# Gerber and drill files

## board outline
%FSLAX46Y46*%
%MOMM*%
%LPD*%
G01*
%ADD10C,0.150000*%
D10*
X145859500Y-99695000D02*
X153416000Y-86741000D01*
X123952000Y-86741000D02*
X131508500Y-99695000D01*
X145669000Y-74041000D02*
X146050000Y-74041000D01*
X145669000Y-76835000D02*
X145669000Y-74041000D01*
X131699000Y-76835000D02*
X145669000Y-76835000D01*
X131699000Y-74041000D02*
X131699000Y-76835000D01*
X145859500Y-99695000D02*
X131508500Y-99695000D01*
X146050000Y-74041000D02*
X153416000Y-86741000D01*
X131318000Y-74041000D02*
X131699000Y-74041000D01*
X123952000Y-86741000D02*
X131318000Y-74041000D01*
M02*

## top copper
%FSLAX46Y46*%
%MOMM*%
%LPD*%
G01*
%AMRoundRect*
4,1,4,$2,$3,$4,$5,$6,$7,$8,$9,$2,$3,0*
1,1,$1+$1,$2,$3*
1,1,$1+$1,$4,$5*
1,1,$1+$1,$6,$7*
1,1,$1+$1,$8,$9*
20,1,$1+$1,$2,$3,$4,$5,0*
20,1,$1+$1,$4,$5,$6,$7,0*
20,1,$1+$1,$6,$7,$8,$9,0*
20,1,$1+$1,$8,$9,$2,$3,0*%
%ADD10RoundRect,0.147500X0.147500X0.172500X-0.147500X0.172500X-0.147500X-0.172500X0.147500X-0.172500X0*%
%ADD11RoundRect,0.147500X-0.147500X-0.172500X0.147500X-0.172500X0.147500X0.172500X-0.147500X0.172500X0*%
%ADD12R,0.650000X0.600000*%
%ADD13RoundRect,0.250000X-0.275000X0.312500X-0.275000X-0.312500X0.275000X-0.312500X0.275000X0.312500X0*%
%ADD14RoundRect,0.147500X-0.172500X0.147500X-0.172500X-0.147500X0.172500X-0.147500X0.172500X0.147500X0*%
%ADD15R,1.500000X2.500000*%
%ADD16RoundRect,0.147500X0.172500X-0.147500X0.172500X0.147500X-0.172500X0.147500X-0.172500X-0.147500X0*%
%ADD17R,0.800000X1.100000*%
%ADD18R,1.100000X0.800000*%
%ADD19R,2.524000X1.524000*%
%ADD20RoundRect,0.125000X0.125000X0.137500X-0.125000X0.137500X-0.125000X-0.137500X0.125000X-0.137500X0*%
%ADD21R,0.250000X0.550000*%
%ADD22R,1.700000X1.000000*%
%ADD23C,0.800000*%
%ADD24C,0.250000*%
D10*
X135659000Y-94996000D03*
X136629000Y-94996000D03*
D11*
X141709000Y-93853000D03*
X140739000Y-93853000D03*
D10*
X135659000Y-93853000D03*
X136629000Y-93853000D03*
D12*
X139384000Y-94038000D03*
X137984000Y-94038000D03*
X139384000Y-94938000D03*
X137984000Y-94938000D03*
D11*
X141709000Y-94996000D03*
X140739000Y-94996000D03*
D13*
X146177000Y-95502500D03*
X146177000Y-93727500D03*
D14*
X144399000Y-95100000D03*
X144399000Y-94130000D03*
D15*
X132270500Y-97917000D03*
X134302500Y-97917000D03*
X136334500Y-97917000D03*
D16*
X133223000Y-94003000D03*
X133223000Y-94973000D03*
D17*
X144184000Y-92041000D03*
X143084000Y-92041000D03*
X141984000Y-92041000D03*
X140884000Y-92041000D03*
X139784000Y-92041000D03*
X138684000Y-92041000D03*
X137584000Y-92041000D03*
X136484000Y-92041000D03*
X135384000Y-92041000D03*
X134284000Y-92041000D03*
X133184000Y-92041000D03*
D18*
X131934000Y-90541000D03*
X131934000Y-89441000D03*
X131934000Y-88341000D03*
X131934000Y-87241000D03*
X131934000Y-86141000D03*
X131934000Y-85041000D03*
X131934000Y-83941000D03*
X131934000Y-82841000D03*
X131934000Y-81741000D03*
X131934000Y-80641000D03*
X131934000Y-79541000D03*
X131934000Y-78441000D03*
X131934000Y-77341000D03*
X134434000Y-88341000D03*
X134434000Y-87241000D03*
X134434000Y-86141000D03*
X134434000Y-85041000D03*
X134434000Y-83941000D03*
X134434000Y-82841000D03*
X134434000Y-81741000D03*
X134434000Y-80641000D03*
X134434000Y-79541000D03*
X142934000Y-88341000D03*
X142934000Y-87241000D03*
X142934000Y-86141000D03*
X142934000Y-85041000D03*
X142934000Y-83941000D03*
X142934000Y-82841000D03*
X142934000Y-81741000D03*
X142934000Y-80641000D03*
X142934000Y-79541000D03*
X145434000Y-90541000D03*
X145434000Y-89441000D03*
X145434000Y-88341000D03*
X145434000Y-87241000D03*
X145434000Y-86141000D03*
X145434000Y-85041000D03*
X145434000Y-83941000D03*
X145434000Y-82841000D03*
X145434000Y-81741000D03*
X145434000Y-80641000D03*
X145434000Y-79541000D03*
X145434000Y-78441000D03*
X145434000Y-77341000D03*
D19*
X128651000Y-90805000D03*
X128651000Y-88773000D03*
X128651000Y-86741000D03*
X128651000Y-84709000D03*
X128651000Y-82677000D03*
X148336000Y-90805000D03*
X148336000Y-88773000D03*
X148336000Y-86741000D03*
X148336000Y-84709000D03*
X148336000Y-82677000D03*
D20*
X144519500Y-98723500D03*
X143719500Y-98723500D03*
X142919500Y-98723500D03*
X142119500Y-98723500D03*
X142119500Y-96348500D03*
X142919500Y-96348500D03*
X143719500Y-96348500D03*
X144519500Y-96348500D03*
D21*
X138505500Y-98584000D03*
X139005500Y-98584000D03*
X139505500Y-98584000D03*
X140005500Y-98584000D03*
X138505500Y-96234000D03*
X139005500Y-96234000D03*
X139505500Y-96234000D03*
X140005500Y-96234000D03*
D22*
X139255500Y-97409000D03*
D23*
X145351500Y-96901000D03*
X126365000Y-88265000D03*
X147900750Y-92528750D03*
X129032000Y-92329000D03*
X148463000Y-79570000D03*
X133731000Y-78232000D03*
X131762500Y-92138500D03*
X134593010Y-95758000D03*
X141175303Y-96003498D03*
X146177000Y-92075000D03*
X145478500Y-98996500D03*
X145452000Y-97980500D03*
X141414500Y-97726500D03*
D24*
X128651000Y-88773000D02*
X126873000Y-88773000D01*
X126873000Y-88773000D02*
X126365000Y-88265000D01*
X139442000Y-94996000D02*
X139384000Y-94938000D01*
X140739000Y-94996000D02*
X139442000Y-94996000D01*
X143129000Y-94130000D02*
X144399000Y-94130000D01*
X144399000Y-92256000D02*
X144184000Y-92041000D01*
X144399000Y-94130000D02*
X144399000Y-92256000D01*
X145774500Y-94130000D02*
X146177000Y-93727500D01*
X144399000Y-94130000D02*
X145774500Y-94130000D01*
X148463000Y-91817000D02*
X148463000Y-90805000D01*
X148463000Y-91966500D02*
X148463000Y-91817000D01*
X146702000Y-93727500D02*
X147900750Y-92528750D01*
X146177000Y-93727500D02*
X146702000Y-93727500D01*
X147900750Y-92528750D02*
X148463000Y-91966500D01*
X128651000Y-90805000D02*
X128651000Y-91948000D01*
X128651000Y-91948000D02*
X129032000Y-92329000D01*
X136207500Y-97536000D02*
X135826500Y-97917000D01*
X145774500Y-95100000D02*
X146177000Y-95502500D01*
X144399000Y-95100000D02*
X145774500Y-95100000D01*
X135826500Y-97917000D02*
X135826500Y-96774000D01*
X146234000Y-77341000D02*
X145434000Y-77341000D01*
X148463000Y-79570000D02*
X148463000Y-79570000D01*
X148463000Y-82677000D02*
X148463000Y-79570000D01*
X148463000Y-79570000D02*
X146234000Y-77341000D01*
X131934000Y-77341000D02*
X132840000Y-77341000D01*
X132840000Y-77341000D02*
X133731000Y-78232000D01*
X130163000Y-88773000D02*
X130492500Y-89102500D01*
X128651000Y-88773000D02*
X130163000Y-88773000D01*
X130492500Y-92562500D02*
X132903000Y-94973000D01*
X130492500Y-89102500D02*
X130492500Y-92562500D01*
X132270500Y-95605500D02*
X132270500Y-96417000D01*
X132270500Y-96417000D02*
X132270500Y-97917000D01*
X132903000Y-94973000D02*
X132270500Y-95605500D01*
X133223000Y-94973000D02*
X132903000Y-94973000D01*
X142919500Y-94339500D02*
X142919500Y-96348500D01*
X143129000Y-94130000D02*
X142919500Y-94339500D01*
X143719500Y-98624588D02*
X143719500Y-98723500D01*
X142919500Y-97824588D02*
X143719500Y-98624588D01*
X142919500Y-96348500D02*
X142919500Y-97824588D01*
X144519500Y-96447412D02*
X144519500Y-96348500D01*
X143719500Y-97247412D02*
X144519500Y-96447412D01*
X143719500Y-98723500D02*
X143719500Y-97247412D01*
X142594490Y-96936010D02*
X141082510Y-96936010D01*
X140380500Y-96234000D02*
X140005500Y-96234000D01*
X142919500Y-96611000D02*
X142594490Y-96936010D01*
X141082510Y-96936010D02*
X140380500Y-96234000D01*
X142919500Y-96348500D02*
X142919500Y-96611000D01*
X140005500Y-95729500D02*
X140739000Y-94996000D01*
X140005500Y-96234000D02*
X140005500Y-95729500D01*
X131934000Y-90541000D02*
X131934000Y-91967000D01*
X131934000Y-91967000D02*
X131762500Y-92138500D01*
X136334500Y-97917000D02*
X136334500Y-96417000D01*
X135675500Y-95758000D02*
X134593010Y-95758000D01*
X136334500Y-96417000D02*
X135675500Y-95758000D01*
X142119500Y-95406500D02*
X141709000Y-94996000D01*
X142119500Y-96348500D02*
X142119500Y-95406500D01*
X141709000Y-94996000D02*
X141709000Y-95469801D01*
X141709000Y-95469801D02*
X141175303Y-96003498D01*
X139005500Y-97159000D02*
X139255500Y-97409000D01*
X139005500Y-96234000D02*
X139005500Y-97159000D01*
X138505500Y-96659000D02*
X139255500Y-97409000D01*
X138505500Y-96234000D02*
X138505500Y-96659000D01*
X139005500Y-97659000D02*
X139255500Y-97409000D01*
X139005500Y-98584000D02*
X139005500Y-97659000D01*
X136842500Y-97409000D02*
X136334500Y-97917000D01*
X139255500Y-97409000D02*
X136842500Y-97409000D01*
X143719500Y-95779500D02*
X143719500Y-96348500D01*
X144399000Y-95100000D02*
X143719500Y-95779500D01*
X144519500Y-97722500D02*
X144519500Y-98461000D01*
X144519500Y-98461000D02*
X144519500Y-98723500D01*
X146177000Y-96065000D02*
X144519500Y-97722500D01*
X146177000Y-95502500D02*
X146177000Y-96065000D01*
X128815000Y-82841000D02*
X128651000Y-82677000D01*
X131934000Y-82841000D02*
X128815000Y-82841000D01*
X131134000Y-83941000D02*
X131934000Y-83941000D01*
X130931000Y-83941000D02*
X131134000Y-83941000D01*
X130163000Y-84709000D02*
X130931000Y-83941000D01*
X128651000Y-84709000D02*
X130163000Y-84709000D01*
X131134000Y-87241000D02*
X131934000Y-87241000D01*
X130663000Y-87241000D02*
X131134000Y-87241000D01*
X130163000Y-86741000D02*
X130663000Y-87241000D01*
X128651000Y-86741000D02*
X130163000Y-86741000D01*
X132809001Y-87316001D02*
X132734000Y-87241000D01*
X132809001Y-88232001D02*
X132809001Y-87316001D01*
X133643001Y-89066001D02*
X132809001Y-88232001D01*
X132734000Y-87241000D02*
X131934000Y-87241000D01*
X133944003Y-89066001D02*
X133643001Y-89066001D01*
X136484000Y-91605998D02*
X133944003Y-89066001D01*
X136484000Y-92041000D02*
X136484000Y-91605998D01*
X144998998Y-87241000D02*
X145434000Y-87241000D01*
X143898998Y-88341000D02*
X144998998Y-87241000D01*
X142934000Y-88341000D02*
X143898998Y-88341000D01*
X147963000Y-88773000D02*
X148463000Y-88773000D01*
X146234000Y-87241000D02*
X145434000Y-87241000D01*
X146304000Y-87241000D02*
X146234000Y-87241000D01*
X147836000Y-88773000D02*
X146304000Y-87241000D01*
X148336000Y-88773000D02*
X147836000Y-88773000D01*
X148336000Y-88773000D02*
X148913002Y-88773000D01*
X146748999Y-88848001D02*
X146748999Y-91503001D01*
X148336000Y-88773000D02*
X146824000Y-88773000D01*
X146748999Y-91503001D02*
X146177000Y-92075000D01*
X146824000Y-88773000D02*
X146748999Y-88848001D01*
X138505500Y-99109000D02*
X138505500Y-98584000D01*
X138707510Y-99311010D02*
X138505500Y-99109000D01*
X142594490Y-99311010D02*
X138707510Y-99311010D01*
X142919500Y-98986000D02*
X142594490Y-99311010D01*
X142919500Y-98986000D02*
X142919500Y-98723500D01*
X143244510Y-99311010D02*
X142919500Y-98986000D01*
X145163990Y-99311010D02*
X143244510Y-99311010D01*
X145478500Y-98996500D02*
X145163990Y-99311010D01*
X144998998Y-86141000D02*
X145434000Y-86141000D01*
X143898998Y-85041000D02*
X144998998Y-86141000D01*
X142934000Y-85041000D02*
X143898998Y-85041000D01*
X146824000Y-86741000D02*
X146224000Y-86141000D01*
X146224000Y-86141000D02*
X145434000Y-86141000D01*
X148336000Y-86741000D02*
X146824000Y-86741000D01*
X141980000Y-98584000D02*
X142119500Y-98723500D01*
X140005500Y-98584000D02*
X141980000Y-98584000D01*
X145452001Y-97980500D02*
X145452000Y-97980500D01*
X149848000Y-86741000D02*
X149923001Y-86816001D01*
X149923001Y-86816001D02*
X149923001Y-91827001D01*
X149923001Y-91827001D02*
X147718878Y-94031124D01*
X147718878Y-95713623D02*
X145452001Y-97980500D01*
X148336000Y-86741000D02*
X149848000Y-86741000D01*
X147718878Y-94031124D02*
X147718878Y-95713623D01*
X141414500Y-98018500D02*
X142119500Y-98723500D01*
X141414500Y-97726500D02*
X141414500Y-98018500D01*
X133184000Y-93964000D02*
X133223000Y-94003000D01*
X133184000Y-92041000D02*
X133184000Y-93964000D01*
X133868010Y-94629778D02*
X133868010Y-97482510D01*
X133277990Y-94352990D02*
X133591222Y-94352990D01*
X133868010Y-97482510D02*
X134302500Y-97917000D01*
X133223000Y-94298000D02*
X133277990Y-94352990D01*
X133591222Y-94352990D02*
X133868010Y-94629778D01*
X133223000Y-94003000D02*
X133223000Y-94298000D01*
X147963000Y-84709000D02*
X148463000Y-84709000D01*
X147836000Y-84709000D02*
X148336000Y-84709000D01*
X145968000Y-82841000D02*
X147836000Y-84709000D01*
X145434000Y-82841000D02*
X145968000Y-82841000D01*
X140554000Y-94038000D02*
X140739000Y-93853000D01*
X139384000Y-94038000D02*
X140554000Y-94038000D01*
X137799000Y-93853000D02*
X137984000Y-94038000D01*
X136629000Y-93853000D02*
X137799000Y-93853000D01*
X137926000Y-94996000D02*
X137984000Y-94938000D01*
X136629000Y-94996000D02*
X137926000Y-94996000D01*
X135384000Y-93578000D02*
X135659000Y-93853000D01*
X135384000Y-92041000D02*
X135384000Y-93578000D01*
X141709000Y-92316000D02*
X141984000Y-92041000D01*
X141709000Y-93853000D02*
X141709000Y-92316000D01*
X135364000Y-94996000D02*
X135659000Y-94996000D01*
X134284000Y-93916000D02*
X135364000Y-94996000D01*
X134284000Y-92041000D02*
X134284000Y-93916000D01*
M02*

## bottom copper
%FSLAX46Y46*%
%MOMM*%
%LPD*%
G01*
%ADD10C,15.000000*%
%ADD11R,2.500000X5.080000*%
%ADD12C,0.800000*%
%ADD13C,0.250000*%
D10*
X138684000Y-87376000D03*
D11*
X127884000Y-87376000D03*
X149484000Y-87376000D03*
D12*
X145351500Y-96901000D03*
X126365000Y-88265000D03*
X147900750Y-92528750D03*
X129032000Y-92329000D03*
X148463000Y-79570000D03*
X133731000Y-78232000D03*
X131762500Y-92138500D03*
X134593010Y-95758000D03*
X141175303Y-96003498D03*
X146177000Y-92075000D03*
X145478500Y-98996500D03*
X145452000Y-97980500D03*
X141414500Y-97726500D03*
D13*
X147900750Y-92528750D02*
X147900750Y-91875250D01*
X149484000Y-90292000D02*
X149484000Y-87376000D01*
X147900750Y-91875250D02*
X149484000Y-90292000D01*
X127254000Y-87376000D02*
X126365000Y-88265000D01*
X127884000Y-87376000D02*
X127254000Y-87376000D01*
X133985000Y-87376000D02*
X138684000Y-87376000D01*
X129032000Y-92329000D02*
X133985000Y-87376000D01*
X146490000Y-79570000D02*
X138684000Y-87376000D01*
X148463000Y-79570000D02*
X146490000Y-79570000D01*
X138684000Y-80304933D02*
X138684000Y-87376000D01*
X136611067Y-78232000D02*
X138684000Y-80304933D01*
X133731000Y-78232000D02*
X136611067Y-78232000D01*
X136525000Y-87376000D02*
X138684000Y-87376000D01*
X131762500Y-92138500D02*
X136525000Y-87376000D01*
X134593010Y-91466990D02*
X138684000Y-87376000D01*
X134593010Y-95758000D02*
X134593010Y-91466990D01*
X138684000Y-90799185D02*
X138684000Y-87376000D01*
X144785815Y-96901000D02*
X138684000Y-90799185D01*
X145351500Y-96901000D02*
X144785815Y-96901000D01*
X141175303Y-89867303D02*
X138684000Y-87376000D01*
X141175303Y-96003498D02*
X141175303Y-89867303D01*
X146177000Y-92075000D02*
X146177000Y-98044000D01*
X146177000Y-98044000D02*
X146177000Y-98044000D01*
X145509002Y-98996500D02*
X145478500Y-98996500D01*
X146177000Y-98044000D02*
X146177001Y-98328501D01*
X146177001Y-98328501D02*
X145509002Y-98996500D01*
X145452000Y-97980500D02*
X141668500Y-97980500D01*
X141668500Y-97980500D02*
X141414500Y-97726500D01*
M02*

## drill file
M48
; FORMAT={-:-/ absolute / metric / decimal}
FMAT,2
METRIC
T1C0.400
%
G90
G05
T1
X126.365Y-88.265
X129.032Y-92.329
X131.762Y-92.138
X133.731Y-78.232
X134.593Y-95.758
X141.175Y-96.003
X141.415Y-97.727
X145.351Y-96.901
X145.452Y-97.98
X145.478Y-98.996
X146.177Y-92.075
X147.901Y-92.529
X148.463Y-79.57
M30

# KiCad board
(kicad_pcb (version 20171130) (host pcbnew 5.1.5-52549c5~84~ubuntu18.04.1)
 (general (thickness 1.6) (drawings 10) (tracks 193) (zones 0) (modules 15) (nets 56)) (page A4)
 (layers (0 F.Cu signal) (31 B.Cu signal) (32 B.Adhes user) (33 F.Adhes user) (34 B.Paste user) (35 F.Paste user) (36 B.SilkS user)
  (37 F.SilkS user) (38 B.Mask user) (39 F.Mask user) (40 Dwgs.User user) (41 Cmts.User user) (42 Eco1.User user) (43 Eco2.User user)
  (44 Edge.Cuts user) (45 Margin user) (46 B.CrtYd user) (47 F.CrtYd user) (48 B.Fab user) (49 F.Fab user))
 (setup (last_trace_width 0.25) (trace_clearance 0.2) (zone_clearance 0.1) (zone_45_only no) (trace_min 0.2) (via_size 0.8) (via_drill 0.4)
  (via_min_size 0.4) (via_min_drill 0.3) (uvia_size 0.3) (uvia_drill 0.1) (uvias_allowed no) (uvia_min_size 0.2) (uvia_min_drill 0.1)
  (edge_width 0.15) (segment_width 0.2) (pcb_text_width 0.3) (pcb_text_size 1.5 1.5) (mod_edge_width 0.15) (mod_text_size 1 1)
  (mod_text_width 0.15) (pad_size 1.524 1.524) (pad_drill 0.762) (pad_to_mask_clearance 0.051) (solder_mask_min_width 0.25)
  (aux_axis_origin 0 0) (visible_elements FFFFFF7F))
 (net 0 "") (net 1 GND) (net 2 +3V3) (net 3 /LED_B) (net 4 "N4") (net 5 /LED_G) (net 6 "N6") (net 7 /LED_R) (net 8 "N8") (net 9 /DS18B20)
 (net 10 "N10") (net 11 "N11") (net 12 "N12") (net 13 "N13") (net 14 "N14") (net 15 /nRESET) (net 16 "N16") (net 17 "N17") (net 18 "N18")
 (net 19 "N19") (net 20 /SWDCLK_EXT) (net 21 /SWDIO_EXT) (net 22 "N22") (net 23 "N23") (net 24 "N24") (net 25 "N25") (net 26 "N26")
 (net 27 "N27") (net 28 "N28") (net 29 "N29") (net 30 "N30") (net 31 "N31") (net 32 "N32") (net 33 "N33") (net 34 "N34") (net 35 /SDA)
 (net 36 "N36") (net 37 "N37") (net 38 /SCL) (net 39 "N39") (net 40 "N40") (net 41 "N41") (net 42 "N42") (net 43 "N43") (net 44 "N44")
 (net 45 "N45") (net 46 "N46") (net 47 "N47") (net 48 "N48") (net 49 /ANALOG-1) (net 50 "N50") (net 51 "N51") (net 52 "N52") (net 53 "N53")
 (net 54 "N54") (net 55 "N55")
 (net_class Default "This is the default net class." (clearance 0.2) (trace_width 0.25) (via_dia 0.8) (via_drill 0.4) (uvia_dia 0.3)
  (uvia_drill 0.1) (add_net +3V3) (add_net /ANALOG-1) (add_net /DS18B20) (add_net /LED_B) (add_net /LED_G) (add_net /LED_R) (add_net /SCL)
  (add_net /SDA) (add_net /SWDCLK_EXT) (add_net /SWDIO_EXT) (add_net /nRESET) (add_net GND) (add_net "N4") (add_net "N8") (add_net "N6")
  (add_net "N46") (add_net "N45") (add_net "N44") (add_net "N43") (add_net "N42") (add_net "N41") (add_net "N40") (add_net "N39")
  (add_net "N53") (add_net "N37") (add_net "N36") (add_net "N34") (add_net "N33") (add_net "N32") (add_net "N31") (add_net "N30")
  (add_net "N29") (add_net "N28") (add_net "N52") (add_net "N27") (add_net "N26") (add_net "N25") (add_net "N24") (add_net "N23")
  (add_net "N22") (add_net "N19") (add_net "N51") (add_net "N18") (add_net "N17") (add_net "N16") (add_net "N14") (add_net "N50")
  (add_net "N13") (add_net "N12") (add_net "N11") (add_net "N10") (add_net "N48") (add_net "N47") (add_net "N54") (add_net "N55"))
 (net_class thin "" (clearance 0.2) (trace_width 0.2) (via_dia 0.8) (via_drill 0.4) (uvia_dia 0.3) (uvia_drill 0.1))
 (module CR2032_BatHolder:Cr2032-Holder (layer B.Cu) (at 138.684 87.376)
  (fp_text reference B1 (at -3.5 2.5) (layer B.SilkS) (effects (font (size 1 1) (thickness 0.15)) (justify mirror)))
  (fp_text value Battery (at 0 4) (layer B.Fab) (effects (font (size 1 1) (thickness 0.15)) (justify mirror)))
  (pad 2 smd circle (at 0 0) (size 15 15) (layers B.Cu B.Mask) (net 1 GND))
  (pad 1 smd rect (at -10.8 0) (size 2.5 5.08) (layers B.Cu B.Paste B.Mask) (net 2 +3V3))
  (pad 1 smd rect (at 10.8 0) (size 2.5 5.08) (layers B.Cu B.Paste B.Mask) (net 2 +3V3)))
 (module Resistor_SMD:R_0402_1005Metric (layer F.Cu) (at 136.144 94.996 180)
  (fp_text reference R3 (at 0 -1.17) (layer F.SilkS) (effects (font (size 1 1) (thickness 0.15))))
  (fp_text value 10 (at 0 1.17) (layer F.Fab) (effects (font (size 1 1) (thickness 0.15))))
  (pad 2 smd roundrect (at 0.485 0 180) (size 0.59 0.64) (layers F.Cu F.Paste F.Mask) (roundrect_rratio 0.25) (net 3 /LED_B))
  (pad 1 smd roundrect (at -0.485 0 180) (size 0.59 0.64) (layers F.Cu F.Paste F.Mask) (roundrect_rratio 0.25) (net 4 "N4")))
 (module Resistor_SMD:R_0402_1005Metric (layer F.Cu) (at 141.224 93.853)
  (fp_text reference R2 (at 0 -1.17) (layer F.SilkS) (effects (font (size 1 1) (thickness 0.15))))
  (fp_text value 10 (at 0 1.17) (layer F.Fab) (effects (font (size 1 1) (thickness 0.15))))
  (pad 2 smd roundrect (at 0.485 0) (size 0.59 0.64) (layers F.Cu F.Paste F.Mask) (roundrect_rratio 0.25) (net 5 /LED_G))
  (pad 1 smd roundrect (at -0.485 0) (size 0.59 0.64) (layers F.Cu F.Paste F.Mask) (roundrect_rratio 0.25) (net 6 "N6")))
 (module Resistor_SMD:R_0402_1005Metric (layer F.Cu) (at 136.144 93.853 180)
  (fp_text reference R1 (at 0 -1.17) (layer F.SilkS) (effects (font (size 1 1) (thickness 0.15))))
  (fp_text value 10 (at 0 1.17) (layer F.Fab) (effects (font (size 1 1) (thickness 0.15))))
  (pad 2 smd roundrect (at 0.485 0 180) (size 0.59 0.64) (layers F.Cu F.Paste F.Mask) (roundrect_rratio 0.25) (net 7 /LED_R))
  (pad 1 smd roundrect (at -0.485 0 180) (size 0.59 0.64) (layers F.Cu F.Paste F.Mask) (roundrect_rratio 0.25) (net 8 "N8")))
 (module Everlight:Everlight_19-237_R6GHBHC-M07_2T (layer F.Cu) (at 138.684 94.488)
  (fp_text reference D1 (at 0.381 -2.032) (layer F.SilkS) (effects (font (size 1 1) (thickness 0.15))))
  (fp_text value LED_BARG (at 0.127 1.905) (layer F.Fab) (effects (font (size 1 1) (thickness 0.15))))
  (pad 4 smd rect (at 0.7 -0.45) (size 0.65 0.6) (layers F.Cu F.Paste F.Mask) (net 6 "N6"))
  (pad 3 smd rect (at -0.7 -0.45) (size 0.65 0.6) (layers F.Cu F.Paste F.Mask) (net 8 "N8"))
  (pad 2 smd rect (at 0.7 0.45) (size 0.65 0.6) (layers F.Cu F.Paste F.Mask) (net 2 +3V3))
  (pad 1 smd rect (at -0.7 0.45) (size 0.65 0.6) (layers F.Cu F.Paste F.Mask) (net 4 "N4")))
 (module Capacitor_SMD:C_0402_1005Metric (layer F.Cu) (at 141.224 94.996)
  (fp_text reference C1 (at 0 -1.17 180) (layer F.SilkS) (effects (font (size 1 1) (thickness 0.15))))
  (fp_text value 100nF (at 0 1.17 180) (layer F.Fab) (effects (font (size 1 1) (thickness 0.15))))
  (pad 2 smd roundrect (at 0.485 0) (size 0.59 0.64) (layers F.Cu F.Paste F.Mask) (roundrect_rratio 0.25) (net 1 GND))
  (pad 1 smd roundrect (at -0.485 0) (size 0.59 0.64) (layers F.Cu F.Paste F.Mask) (roundrect_rratio 0.25) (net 2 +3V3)))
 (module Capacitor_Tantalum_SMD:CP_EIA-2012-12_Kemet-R (layer F.Cu) (at 146.177 94.615 270)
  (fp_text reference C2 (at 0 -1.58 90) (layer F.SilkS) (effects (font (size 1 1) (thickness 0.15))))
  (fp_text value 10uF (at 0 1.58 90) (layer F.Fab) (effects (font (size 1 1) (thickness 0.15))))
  (pad 2 smd roundrect (at 0.8875 0 270) (size 1.125 1.05) (layers F.Cu F.Paste F.Mask) (roundrect_rratio 0.238095) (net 1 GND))
  (pad 1 smd roundrect (at -0.8875 0 270) (size 1.125 1.05) (layers F.Cu F.Paste F.Mask) (roundrect_rratio 0.238095) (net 2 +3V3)))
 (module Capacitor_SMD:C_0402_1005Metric (layer F.Cu) (at 144.399 94.615 270)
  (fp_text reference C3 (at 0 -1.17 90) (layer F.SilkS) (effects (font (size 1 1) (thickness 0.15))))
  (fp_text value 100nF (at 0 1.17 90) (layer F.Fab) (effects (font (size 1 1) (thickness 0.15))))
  (pad 2 smd roundrect (at 0.485 0 270) (size 0.59 0.64) (layers F.Cu F.Paste F.Mask) (roundrect_rratio 0.25) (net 1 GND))
  (pad 1 smd roundrect (at -0.485 0 270) (size 0.59 0.64) (layers F.Cu F.Paste F.Mask) (roundrect_rratio 0.25) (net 2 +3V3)))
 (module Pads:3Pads (layer F.Cu) (at 134.3025 100.457 180)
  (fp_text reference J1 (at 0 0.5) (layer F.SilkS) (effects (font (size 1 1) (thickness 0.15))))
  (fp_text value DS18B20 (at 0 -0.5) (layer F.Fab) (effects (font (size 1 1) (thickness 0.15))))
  (pad 3 smd rect (at 2.032 2.54 180) (size 1.5 2.5) (layers F.Cu F.Paste F.Mask) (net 2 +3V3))
  (pad 2 smd rect (at 0 2.54 180) (size 1.5 2.5) (layers F.Cu F.Paste F.Mask) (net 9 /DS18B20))
  (pad 1 smd rect (at -2.032 2.54 180) (size 1.5 2.5) (layers F.Cu F.Paste F.Mask) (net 1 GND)))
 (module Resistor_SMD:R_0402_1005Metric (layer F.Cu) (at 133.223 94.488 90)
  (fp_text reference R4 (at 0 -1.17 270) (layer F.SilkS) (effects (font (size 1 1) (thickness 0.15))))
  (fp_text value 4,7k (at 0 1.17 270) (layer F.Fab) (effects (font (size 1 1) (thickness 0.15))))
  (pad 2 smd roundrect (at 0.485 0 90) (size 0.59 0.64) (layers F.Cu F.Paste F.Mask) (roundrect_rratio 0.25) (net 9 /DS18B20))
  (pad 1 smd roundrect (at -0.485 0 90) (size 0.59 0.64) (layers F.Cu F.Paste F.Mask) (roundrect_rratio 0.25) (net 2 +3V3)))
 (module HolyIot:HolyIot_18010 (layer F.Cu) (at 138.684 74.041)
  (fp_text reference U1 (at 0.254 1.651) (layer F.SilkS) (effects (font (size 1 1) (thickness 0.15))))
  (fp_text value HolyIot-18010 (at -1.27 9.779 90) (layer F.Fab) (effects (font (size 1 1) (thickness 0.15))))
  (pad 55 smd rect (at 5.5 18) (size 0.8 1.1) (layers F.Cu F.Paste F.Mask) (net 2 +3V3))
  (pad 54 smd rect (at 4.4 18) (size 0.8 1.1) (layers F.Cu F.Paste F.Mask) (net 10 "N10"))
  (pad 53 smd rect (at 3.3 18) (size 0.8 1.1) (layers F.Cu F.Paste F.Mask) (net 5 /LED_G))
  (pad 52 smd rect (at 2.2 18) (size 0.8 1.1) (layers F.Cu F.Paste F.Mask) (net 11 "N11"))
  (pad 51 smd rect (at 1.1 18) (size 0.8 1.1) (layers F.Cu F.Paste F.Mask) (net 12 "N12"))
  (pad 50 smd rect (at 0 18) (size 0.8 1.1) (layers F.Cu F.Paste F.Mask) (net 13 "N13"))
  (pad 49 smd rect (at -1.1 18) (size 0.8 1.1) (layers F.Cu F.Paste F.Mask) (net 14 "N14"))
  (pad 48 smd rect (at -2.2 18) (size 0.8 1.1) (layers F.Cu F.Paste F.Mask) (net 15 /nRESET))
  (pad 47 smd rect (at -3.3 18) (size 0.8 1.1) (layers F.Cu F.Paste F.Mask) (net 7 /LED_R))
  (pad 46 smd rect (at -4.4 18) (size 0.8 1.1) (layers F.Cu F.Paste F.Mask) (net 3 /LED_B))
  (pad 45 smd rect (at -5.5 18) (size 0.8 1.1) (layers F.Cu F.Paste F.Mask) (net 9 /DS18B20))
  (pad 44 smd rect (at -6.75 16.5) (size 1.1 0.8) (layers F.Cu F.Paste F.Mask) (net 1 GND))
  (pad 43 smd rect (at -6.75 15.4) (size 1.1 0.8) (layers F.Cu F.Paste F.Mask) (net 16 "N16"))
  (pad 42 smd rect (at -6.75 14.3) (size 1.1 0.8) (layers F.Cu F.Paste F.Mask) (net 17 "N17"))
  (pad 41 smd rect (at -6.75 13.2) (size 1.1 0.8) (layers F.Cu F.Paste F.Mask) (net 15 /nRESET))
  (pad 40 smd rect (at -6.75 12.1) (size 1.1 0.8) (layers F.Cu F.Paste F.Mask) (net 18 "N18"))
  (pad 39 smd rect (at -6.75 11) (size 1.1 0.8) (layers F.Cu F.Paste F.Mask) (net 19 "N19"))
  (pad 38 smd rect (at -6.75 9.9) (size 1.1 0.8) (layers F.Cu F.Paste F.Mask) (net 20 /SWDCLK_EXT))
  (pad 37 smd rect (at -6.75 8.8) (size 1.1 0.8) (layers F.Cu F.Paste F.Mask) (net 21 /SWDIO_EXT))
  (pad 36 smd rect (at -6.75 7.7) (size 1.1 0.8) (layers F.Cu F.Paste F.Mask) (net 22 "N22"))
  (pad 35 smd rect (at -6.75 6.6) (size 1.1 0.8) (layers F.Cu F.Paste F.Mask) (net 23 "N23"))
  (pad 34 smd rect (at -6.75 5.5) (size 1.1 0.8) (layers F.Cu F.Paste F.Mask) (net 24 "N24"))
  (pad 33 smd rect (at -6.75 4.4) (size 1.1 0.8) (layers F.Cu F.Paste F.Mask) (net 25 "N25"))
  (pad 32 smd rect (at -6.75 3.3) (size 1.1 0.8) (layers F.Cu F.Paste F.Mask) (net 1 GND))
  (pad 31 smd rect (at -4.25 14.3) (size 1.1 0.8) (layers F.Cu F.Paste F.Mask) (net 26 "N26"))
  (pad 30 smd rect (at -4.25 13.2) (size 1.1 0.8) (layers F.Cu F.Paste F.Mask) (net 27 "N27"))
  (pad 29 smd rect (at -4.25 12.1) (size 1.1 0.8) (layers F.Cu F.Paste F.Mask) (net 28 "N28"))
  (pad 28 smd rect (at -4.25 11) (size 1.1 0.8) (layers F.Cu F.Paste F.Mask) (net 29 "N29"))
  (pad 27 smd rect (at -4.25 9.9) (size 1.1 0.8) (layers F.Cu F.Paste F.Mask) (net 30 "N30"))
  (pad 26 smd rect (at -4.25 8.8) (size 1.1 0.8) (layers F.Cu F.Paste F.Mask) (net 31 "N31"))
  (pad 25 smd rect (at -4.25 7.7) (size 1.1 0.8) (layers F.Cu F.Paste F.Mask) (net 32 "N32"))
  (pad 24 smd rect (at -4.25 6.6) (size 1.1 0.8) (layers F.Cu F.Paste F.Mask) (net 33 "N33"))
  (pad 23 smd rect (at -4.25 5.5) (size 1.1 0.8) (layers F.Cu F.Paste F.Mask) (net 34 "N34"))
  (pad 22 smd rect (at 4.25 14.3) (size 1.1 0.8) (layers F.Cu F.Paste F.Mask) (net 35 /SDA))
  (pad 21 smd rect (at 4.25 13.2) (size 1.1 0.8) (layers F.Cu F.Paste F.Mask) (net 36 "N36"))
  (pad 20 smd rect (at 4.25 12.1) (size 1.1 0.8) (layers F.Cu F.Paste F.Mask) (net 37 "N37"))
  (pad 19 smd rect (at 4.25 11) (size 1.1 0.8) (layers F.Cu F.Paste F.Mask) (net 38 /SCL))
  (pad 18 smd rect (at 4.25 9.9) (size 1.1 0.8) (layers F.Cu F.Paste F.Mask) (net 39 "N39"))
  (pad 17 smd rect (at 4.25 8.8) (size 1.1 0.8) (layers F.Cu F.Paste F.Mask) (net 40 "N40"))
  (pad 16 smd rect (at 4.25 7.7) (size 1.1 0.8) (layers F.Cu F.Paste F.Mask) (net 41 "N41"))
  (pad 15 smd rect (at 4.25 6.6) (size 1.1 0.8) (layers F.Cu F.Paste F.Mask) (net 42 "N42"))
  (pad 14 smd rect (at 4.25 5.5) (size 1.1 0.8) (layers F.Cu F.Paste F.Mask) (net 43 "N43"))
  (pad 13 smd rect (at 6.75 16.5) (size 1.1 0.8) (layers F.Cu F.Paste F.Mask) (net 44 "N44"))
  (pad 12 smd rect (at 6.75 15.4) (size 1.1 0.8) (layers F.Cu F.Paste F.Mask) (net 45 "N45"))
  (pad 11 smd rect (at 6.75 14.3) (size 1.1 0.8) (layers F.Cu F.Paste F.Mask) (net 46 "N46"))
  (pad 10 smd rect (at 6.75 13.2) (size 1.1 0.8) (layers F.Cu F.Paste F.Mask) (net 35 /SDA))
  (pad 9 smd rect (at 6.75 12.1) (size 1.1 0.8) (layers F.Cu F.Paste F.Mask) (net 38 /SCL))
  (pad 8 smd rect (at 6.75 11) (size 1.1 0.8) (layers F.Cu F.Paste F.Mask) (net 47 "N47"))
  (pad 7 smd rect (at 6.75 9.9) (size 1.1 0.8) (layers F.Cu F.Paste F.Mask) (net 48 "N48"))
  (pad 6 smd rect (at 6.75 8.8) (size 1.1 0.8) (layers F.Cu F.Paste F.Mask) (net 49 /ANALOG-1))
  (pad 5 smd rect (at 6.75 7.7) (size 1.1 0.8) (layers F.Cu F.Paste F.Mask) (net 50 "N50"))
  (pad 4 smd rect (at 6.75 6.6) (size 1.1 0.8) (layers F.Cu F.Paste F.Mask) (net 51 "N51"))
  (pad 3 smd rect (at 6.75 5.5) (size 1.1 0.8) (layers F.Cu F.Paste F.Mask) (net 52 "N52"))
  (pad 2 smd rect (at 6.75 4.4) (size 1.1 0.8) (layers F.Cu F.Paste F.Mask) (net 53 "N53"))
  (pad 1 smd rect (at 6.75 3.3) (size 1.1 0.8) (layers F.Cu F.Paste F.Mask) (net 1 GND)))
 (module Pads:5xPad (layer F.Cu) (at 128.651 82.677)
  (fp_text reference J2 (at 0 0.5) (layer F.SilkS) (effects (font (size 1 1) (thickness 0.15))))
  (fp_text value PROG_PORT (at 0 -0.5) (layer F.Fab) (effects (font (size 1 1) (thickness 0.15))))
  (pad 5 smd rect (at 0 8.128) (size 2.524 1.524) (layers F.Cu F.Paste F.Mask) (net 1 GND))
  (pad 4 smd rect (at 0 6.096) (size 2.524 1.524) (layers F.Cu F.Paste F.Mask) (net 2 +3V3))
  (pad 3 smd rect (at 0 4.064) (size 2.524 1.524) (layers F.Cu F.Paste F.Mask) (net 15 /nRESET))
  (pad 2 smd rect (at 0 2.032) (size 2.524 1.524) (layers F.Cu F.Paste F.Mask) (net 20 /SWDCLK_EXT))
  (pad 1 smd rect (at 0 0) (size 2.524 1.524) (layers F.Cu F.Paste F.Mask) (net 21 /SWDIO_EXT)))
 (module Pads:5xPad (layer F.Cu) (at 148.336 82.677)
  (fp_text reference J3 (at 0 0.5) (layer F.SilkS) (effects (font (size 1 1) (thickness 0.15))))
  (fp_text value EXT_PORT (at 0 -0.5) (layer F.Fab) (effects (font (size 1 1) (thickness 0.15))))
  (pad 5 smd rect (at 0 8.128) (size 2.524 1.524) (layers F.Cu F.Paste F.Mask) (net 2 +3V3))
  (pad 4 smd rect (at 0 6.096) (size 2.524 1.524) (layers F.Cu F.Paste F.Mask) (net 35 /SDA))
  (pad 3 smd rect (at 0 4.064) (size 2.524 1.524) (layers F.Cu F.Paste F.Mask) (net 38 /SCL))
  (pad 2 smd rect (at 0 2.032) (size 2.524 1.524) (layers F.Cu F.Paste F.Mask) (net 49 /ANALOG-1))
  (pad 1 smd rect (at 0 0) (size 2.524 1.524) (layers F.Cu F.Paste F.Mask) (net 1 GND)))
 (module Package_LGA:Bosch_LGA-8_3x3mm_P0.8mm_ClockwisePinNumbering (layer F.Cu) (at 143.3195 97.536 180)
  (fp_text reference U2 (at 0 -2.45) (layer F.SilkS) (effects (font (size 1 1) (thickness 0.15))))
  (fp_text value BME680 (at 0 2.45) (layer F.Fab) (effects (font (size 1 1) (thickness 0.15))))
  (pad 1 smd roundrect (at -1.2 -1.1875 180) (size 0.5 0.525) (layers F.Cu F.Paste F.Mask) (roundrect_rratio 0.25) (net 1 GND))
  (pad 2 smd roundrect (at -0.4 -1.1875 180) (size 0.5 0.525) (layers F.Cu F.Paste F.Mask) (roundrect_rratio 0.25) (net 2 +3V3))
  (pad 3 smd roundrect (at 0.4 -1.1875 180) (size 0.5 0.525) (layers F.Cu F.Paste F.Mask) (roundrect_rratio 0.25) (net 35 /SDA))
  (pad 4 smd roundrect (at 1.2 -1.1875 180) (size 0.5 0.525) (layers F.Cu F.Paste F.Mask) (roundrect_rratio 0.25) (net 38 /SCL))
  (pad 5 smd roundrect (at 1.2 1.1875 180) (size 0.5 0.525) (layers F.Cu F.Paste F.Mask) (roundrect_rratio 0.25) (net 1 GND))
  (pad 6 smd roundrect (at 0.4 1.1875 180) (size 0.5 0.525) (layers F.Cu F.Paste F.Mask) (roundrect_rratio 0.25) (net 2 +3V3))
  (pad 7 smd roundrect (at -0.4 1.1875 180) (size 0.5 0.525) (layers F.Cu F.Paste F.Mask) (roundrect_rratio 0.25) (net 1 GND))
  (pad 8 smd roundrect (at -1.2 1.1875 180) (size 0.5 0.525) (layers F.Cu F.Paste F.Mask) (roundrect_rratio 0.25) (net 2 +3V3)))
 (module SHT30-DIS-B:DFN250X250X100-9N (layer F.Cu) (at 139.2555 97.409 90)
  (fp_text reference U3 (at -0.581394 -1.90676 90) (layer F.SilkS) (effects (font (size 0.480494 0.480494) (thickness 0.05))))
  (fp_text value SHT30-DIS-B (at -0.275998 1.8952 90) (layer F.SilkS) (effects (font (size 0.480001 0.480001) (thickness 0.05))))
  (pad 1 smd rect (at -1.175 -0.75 90) (size 0.55 0.25) (layers F.Cu F.Paste F.Mask) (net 35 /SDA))
  (pad 2 smd rect (at -1.175 -0.25 90) (size 0.55 0.25) (layers F.Cu F.Paste F.Mask) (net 1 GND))
  (pad 3 smd rect (at -1.175 0.25 90) (size 0.55 0.25) (layers F.Cu F.Paste F.Mask) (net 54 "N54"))
  (pad 4 smd rect (at -1.175 0.75 90) (size 0.55 0.25) (layers F.Cu F.Paste F.Mask) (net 38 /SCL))
  (pad 8 smd rect (at 1.175 -0.75 90) (size 0.55 0.25) (layers F.Cu F.Paste F.Mask) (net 1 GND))
  (pad 7 smd rect (at 1.175 -0.25 90) (size 0.55 0.25) (layers F.Cu F.Paste F.Mask) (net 1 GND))
  (pad 6 smd rect (at 1.175 0.25 90) (size 0.55 0.25) (layers F.Cu F.Paste F.Mask) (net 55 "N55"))
  (pad 5 smd rect (at 1.175 0.75 90) (size 0.55 0.25) (layers F.Cu F.Paste F.Mask) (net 2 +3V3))
  (pad 9 smd rect (at 0 0 90) (size 1 1.7) (layers F.Cu F.Paste F.Mask) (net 1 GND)))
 (gr_line (start 145.8595 99.695) (end 153.416 86.741) (layer Edge.Cuts) (width 0.15))
 (gr_line (start 123.952 86.741) (end 131.5085 99.695) (layer Edge.Cuts) (width 0.15))
 (gr_line (start 145.669 74.041) (end 146.05 74.041) (layer Edge.Cuts) (width 0.15))
 (gr_line (start 145.669 76.835) (end 145.669 74.041) (layer Edge.Cuts) (width 0.15))
 (gr_line (start 131.699 76.835) (end 145.669 76.835) (layer Edge.Cuts) (width 0.15))
 (gr_line (start 131.699 74.041) (end 131.699 76.835) (layer Edge.Cuts) (width 0.15))
 (gr_line (start 145.8595 99.695) (end 131.5085 99.695) (layer Edge.Cuts) (width 0.15))
 (gr_line (start 146.05 74.041) (end 153.416 86.741) (layer Edge.Cuts) (width 0.15))
 (gr_line (start 131.318 74.041) (end 131.699 74.041) (layer Edge.Cuts) (width 0.15))
 (gr_line (start 123.952 86.741) (end 131.318 74.041) (layer Edge.Cuts) (width 0.15))
 (via (at 145.3515 96.901) (size 0.8) (drill 0.4) (layers F.Cu B.Cu) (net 1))
 (segment (start 128.651 88.773) (end 126.873 88.773) (width 0.25) (layer F.Cu) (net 2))
 (via (at 126.365 88.265) (size 0.8) (drill 0.4) (layers F.Cu B.Cu) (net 2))
 (segment (start 126.873 88.773) (end 126.365 88.265) (width 0.25) (layer F.Cu) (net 2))
 (segment (start 139.442 94.996) (end 139.384 94.938) (width 0.25) (layer F.Cu) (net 2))
 (segment (start 140.739 94.996) (end 139.442 94.996) (width 0.25) (layer F.Cu) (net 2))
 (segment (start 143.129 94.13) (end 144.399 94.13) (width 0.25) (layer F.Cu) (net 2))
 (segment (start 144.399 92.256) (end 144.184 92.041) (width 0.25) (layer F.Cu) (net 2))
 (segment (start 144.399 94.13) (end 144.399 92.256) (width 0.25) (layer F.Cu) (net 2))
 (segment (start 145.7745 94.13) (end 146.177 93.7275) (width 0.25) (layer F.Cu) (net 2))
 (segment (start 144.399 94.13) (end 145.7745 94.13) (width 0.25) (layer F.Cu) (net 2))
 (segment (start 148.463 91.817) (end 148.463 90.805) (width 0.25) (layer F.Cu) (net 2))
 (segment (start 148.463 91.9665) (end 148.463 91.817) (width 0.25) (layer F.Cu) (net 2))
 (segment (start 146.702 93.7275) (end 147.90075 92.52875) (width 0.25) (layer F.Cu) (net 2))
 (segment (start 146.177 93.7275) (end 146.702 93.7275) (width 0.25) (layer F.Cu) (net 2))
 (segment (start 147.90075 92.52875) (end 148.463 91.9665) (width 0.25) (layer F.Cu) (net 2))
 (via (at 147.90075 92.52875) (size 0.8) (drill 0.4) (layers F.Cu B.Cu) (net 2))
 (segment (start 147.90075 92.52875) (end 147.90075 91.87525) (width 0.25) (layer B.Cu) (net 2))
 (segment (start 149.484 90.292) (end 149.484 87.376) (width 0.25) (layer B.Cu) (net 2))
 (segment (start 147.90075 91.87525) (end 149.484 90.292) (width 0.25) (layer B.Cu) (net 2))
 (segment (start 127.254 87.376) (end 126.365 88.265) (width 0.25) (layer B.Cu) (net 2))
 (segment (start 127.884 87.376) (end 127.254 87.376) (width 0.25) (layer B.Cu) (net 2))
 (via (at 129.032 92.329) (size 0.8) (drill 0.4) (layers F.Cu B.Cu) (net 1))
 (segment (start 128.651 90.805) (end 128.651 91.948) (width 0.25) (layer F.Cu) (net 1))
 (segment (start 128.651 91.948) (end 129.032 92.329) (width 0.25) (layer F.Cu) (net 1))
 (segment (start 133.985 87.376) (end 138.684 87.376) (width 0.25) (layer B.Cu) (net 1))
 (segment (start 129.032 92.329) (end 133.985 87.376) (width 0.25) (layer B.Cu) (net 1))
 (segment (start 136.2075 97.536) (end 135.8265 97.917) (width 0.25) (layer F.Cu) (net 1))
 (segment (start 145.7745 95.1) (end 146.177 95.5025) (width 0.25) (layer F.Cu) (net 1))
 (segment (start 144.399 95.1) (end 145.7745 95.1) (width 0.25) (layer F.Cu) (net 1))
 (segment (start 135.8265 97.917) (end 135.8265 96.774) (width 0.25) (layer F.Cu) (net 1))
 (segment (start 146.234 77.341) (end 145.434 77.341) (width 0.25) (layer F.Cu) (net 1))
 (segment (start 148.463 79.57) (end 148.463 79.57) (width 0.25) (layer F.Cu) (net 1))
 (segment (start 148.463 82.677) (end 148.463 79.57) (width 0.25) (layer F.Cu) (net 1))
 (segment (start 148.463 79.57) (end 146.234 77.341) (width 0.25) (layer F.Cu) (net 1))
 (via (at 148.463 79.57) (size 0.8) (drill 0.4) (layers F.Cu B.Cu) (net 1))
 (segment (start 146.49 79.57) (end 138.684 87.376) (width 0.25) (layer B.Cu) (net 1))
 (segment (start 148.463 79.57) (end 146.49 79.57) (width 0.25) (layer B.Cu) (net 1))
 (via (at 133.731 78.232) (size 0.8) (drill 0.4) (layers F.Cu B.Cu) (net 1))
 (segment (start 131.934 77.341) (end 132.84 77.341) (width 0.25) (layer F.Cu) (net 1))
 (segment (start 132.84 77.341) (end 133.731 78.232) (width 0.25) (layer F.Cu) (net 1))
 (segment (start 138.684 80.304933) (end 138.684 87.376) (width 0.25) (layer B.Cu) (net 1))
 (segment (start 136.611067 78.232) (end 138.684 80.304933) (width 0.25) (layer B.Cu) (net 1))
 (segment (start 133.731 78.232) (end 136.611067 78.232) (width 0.25) (layer B.Cu) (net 1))
 (segment (start 130.163 88.773) (end 130.4925 89.1025) (width 0.25) (layer F.Cu) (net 2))
 (segment (start 128.651 88.773) (end 130.163 88.773) (width 0.25) (layer F.Cu) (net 2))
 (segment (start 130.4925 92.5625) (end 132.903 94.973) (width 0.25) (layer F.Cu) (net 2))
 (segment (start 130.4925 89.1025) (end 130.4925 92.5625) (width 0.25) (layer F.Cu) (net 2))
 (segment (start 132.2705 95.6055) (end 132.2705 96.417) (width 0.25) (layer F.Cu) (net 2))
 (segment (start 132.2705 96.417) (end 132.2705 97.917) (width 0.25) (layer F.Cu) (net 2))
 (segment (start 132.903 94.973) (end 132.2705 95.6055) (width 0.25) (layer F.Cu) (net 2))
 (segment (start 133.223 94.973) (end 132.903 94.973) (width 0.25) (layer F.Cu) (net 2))
 (segment (start 142.9195 94.3395) (end 142.9195 96.3485) (width 0.25) (layer F.Cu) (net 2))
 (segment (start 143.129 94.13) (end 142.9195 94.3395) (width 0.25) (layer F.Cu) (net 2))
 (segment (start 143.7195 98.624588) (end 143.7195 98.7235) (width 0.25) (layer F.Cu) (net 2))
 (segment (start 142.9195 97.824588) (end 143.7195 98.624588) (width 0.25) (layer F.Cu) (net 2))
 (segment (start 142.9195 96.3485) (end 142.9195 97.824588) (width 0.25) (layer F.Cu) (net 2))
 (segment (start 144.5195 96.447412) (end 144.5195 96.3485) (width 0.25) (layer F.Cu) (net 2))
 (segment (start 143.7195 97.247412) (end 144.5195 96.447412) (width 0.25) (layer F.Cu) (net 2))
 (segment (start 143.7195 98.7235) (end 143.7195 97.247412) (width 0.25) (layer F.Cu) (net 2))
 (segment (start 142.59449 96.93601) (end 141.08251 96.93601) (width 0.25) (layer F.Cu) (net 2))
 (segment (start 140.3805 96.234) (end 140.0055 96.234) (width 0.25) (layer F.Cu) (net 2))
 (segment (start 142.9195 96.611) (end 142.59449 96.93601) (width 0.25) (layer F.Cu) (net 2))
 (segment (start 141.08251 96.93601) (end 140.3805 96.234) (width 0.25) (layer F.Cu) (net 2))
 (segment (start 142.9195 96.3485) (end 142.9195 96.611) (width 0.25) (layer F.Cu) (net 2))
 (segment (start 140.0055 95.7295) (end 140.739 94.996) (width 0.25) (layer F.Cu) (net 2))
 (segment (start 140.0055 96.234) (end 140.0055 95.7295) (width 0.25) (layer F.Cu) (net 2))
 (via (at 131.7625 92.1385) (size 0.8) (drill 0.4) (layers F.Cu B.Cu) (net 1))
 (segment (start 131.934 90.541) (end 131.934 91.967) (width 0.25) (layer F.Cu) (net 1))
 (segment (start 131.934 91.967) (end 131.7625 92.1385) (width 0.25) (layer F.Cu) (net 1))
 (segment (start 136.525 87.376) (end 138.684 87.376) (width 0.25) (layer B.Cu) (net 1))
 (segment (start 131.7625 92.1385) (end 136.525 87.376) (width 0.25) (layer B.Cu) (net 1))
 (via (at 134.59301 95.758) (size 0.8) (drill 0.4) (layers F.Cu B.Cu) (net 1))
 (segment (start 136.3345 97.917) (end 136.3345 96.417) (width 0.25) (layer F.Cu) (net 1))
 (segment (start 135.6755 95.758) (end 134.59301 95.758) (width 0.25) (layer F.Cu) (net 1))
 (segment (start 136.3345 96.417) (end 135.6755 95.758) (width 0.25) (layer F.Cu) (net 1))
 (segment (start 134.59301 91.46699) (end 138.684 87.376) (width 0.25) (layer B.Cu) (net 1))
 (segment (start 134.59301 95.758) (end 134.59301 91.46699) (width 0.25) (layer B.Cu) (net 1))
 (segment (start 142.1195 95.4065) (end 141.709 94.996) (width 0.25) (layer F.Cu) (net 1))
 (segment (start 142.1195 96.3485) (end 142.1195 95.4065) (width 0.25) (layer F.Cu) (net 1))
 (via (at 141.175303 96.003498) (size 0.8) (drill 0.4) (layers F.Cu B.Cu) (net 1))
 (segment (start 141.709 94.996) (end 141.709 95.469801) (width 0.25) (layer F.Cu) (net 1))
 (segment (start 141.709 95.469801) (end 141.175303 96.003498) (width 0.25) (layer F.Cu) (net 1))
 (segment (start 139.0055 97.159) (end 139.2555 97.409) (width 0.25) (layer F.Cu) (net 1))
 (segment (start 139.0055 96.234) (end 139.0055 97.159) (width 0.25) (layer F.Cu) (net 1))
 (segment (start 138.5055 96.659) (end 139.2555 97.409) (width 0.25) (layer F.Cu) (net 1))
 (segment (start 138.5055 96.234) (end 138.5055 96.659) (width 0.25) (layer F.Cu) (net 1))
 (segment (start 139.0055 97.659) (end 139.2555 97.409) (width 0.25) (layer F.Cu) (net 1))
 (segment (start 139.0055 98.584) (end 139.0055 97.659) (width 0.25) (layer F.Cu) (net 1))
 (segment (start 136.8425 97.409) (end 136.3345 97.917) (width 0.25) (layer F.Cu) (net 1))
 (segment (start 139.2555 97.409) (end 136.8425 97.409) (width 0.25) (layer F.Cu) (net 1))
 (segment (start 143.7195 95.7795) (end 143.7195 96.3485) (width 0.25) (layer F.Cu) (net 1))
 (segment (start 144.399 95.1) (end 143.7195 95.7795) (width 0.25) (layer F.Cu) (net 1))
 (segment (start 144.5195 97.7225) (end 144.5195 98.461) (width 0.25) (layer F.Cu) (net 1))
 (segment (start 144.5195 98.461) (end 144.5195 98.7235) (width 0.25) (layer F.Cu) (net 1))
 (segment (start 146.177 96.065) (end 144.5195 97.7225) (width 0.25) (layer F.Cu) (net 1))
 (segment (start 146.177 95.5025) (end 146.177 96.065) (width 0.25) (layer F.Cu) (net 1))
 (segment (start 138.684 90.799185) (end 138.684 87.376) (width 0.25) (layer B.Cu) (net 1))
 (segment (start 144.785815 96.901) (end 138.684 90.799185) (width 0.25) (layer B.Cu) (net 1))
 (segment (start 145.3515 96.901) (end 144.785815 96.901) (width 0.25) (layer B.Cu) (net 1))
 (segment (start 141.175303 89.867303) (end 138.684 87.376) (width 0.25) (layer B.Cu) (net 1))
 (segment (start 141.175303 96.003498) (end 141.175303 89.867303) (width 0.25) (layer B.Cu) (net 1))
 (segment (start 128.815 82.841) (end 128.651 82.677) (width 0.25) (layer F.Cu) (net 21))
 (segment (start 131.934 82.841) (end 128.815 82.841) (width 0.25) (layer F.Cu) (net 21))
 (segment (start 131.134 83.941) (end 131.934 83.941) (width 0.25) (layer F.Cu) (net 20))
 (segment (start 130.931 83.941) (end 131.134 83.941) (width 0.25) (layer F.Cu) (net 20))
 (segment (start 130.163 84.709) (end 130.931 83.941) (width 0.25) (layer F.Cu) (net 20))
 (segment (start 128.651 84.709) (end 130.163 84.709) (width 0.25) (layer F.Cu) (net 20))
 (segment (start 131.134 87.241) (end 131.934 87.241) (width 0.25) (layer F.Cu) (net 15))
 (segment (start 130.663 87.241) (end 131.134 87.241) (width 0.25) (layer F.Cu) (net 15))
 (segment (start 130.163 86.741) (end 130.663 87.241) (width 0.25) (layer F.Cu) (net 15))
 (segment (start 128.651 86.741) (end 130.163 86.741) (width 0.25) (layer F.Cu) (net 15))
 (segment (start 132.809001 87.316001) (end 132.734 87.241) (width 0.25) (layer F.Cu) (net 15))
 (segment (start 132.809001 88.232001) (end 132.809001 87.316001) (width 0.25) (layer F.Cu) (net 15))
 (segment (start 133.643001 89.066001) (end 132.809001 88.232001) (width 0.25) (layer F.Cu) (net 15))
 (segment (start 132.734 87.241) (end 131.934 87.241) (width 0.25) (layer F.Cu) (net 15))
 (segment (start 133.944003 89.066001) (end 133.643001 89.066001) (width 0.25) (layer F.Cu) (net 15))
 (segment (start 136.484 91.605998) (end 133.944003 89.066001) (width 0.25) (layer F.Cu) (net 15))
 (segment (start 136.484 92.041) (end 136.484 91.605998) (width 0.25) (layer F.Cu) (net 15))
 (segment (start 144.998998 87.241) (end 145.434 87.241) (width 0.25) (layer F.Cu) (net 35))
 (segment (start 143.898998 88.341) (end 144.998998 87.241) (width 0.25) (layer F.Cu) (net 35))
 (segment (start 142.934 88.341) (end 143.898998 88.341) (width 0.25) (layer F.Cu) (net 35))
 (segment (start 147.963 88.773) (end 148.463 88.773) (width 0.25) (layer F.Cu) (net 35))
 (segment (start 146.234 87.241) (end 145.434 87.241) (width 0.25) (layer F.Cu) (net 35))
 (segment (start 146.304 87.241) (end 146.234 87.241) (width 0.25) (layer F.Cu) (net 35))
 (segment (start 147.836 88.773) (end 146.304 87.241) (width 0.25) (layer F.Cu) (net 35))
 (segment (start 148.336 88.773) (end 147.836 88.773) (width 0.25) (layer F.Cu) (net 35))
 (segment (start 148.336 88.773) (end 148.913002 88.773) (width 0.25) (layer F.Cu) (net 35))
 (via (at 146.177 92.075) (size 0.8) (drill 0.4) (layers F.Cu B.Cu) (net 35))
 (segment (start 146.748999 88.848001) (end 146.748999 91.503001) (width 0.25) (layer F.Cu) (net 35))
 (segment (start 148.336 88.773) (end 146.824 88.773) (width 0.25) (layer F.Cu) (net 35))
 (segment (start 146.748999 91.503001) (end 146.177 92.075) (width 0.25) (layer F.Cu) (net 35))
 (segment (start 146.824 88.773) (end 146.748999 88.848001) (width 0.25) (layer F.Cu) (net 35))
 (segment (start 146.177 92.075) (end 146.177 98.044) (width 0.25) (layer B.Cu) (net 35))
 (segment (start 146.177 98.044) (end 146.177 98.044) (width 0.25) (layer B.Cu) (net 35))
 (segment (start 138.5055 99.109) (end 138.5055 98.584) (width 0.25) (layer F.Cu) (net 35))
 (segment (start 138.70751 99.31101) (end 138.5055 99.109) (width 0.25) (layer F.Cu) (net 35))
 (segment (start 142.59449 99.31101) (end 138.70751 99.31101) (width 0.25) (layer F.Cu) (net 35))
 (segment (start 142.9195 98.986) (end 142.59449 99.31101) (width 0.25) (layer F.Cu) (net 35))
 (segment (start 145.509002 98.9965) (end 145.4785 98.9965) (width 0.25) (layer B.Cu) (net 35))
 (segment (start 146.177 98.044) (end 146.177001 98.328501) (width 0.25) (layer B.Cu) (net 35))
 (via (at 145.4785 98.9965) (size 0.8) (drill 0.4) (layers F.Cu B.Cu) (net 35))
 (segment (start 146.177001 98.328501) (end 145.509002 98.9965) (width 0.25) (layer B.Cu) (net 35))
 (segment (start 142.9195 98.986) (end 142.9195 98.7235) (width 0.25) (layer F.Cu) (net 35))
 (segment (start 143.24451 99.31101) (end 142.9195 98.986) (width 0.25) (layer F.Cu) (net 35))
 (segment (start 145.16399 99.31101) (end 143.24451 99.31101) (width 0.25) (layer F.Cu) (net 35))
 (segment (start 145.4785 98.9965) (end 145.16399 99.31101) (width 0.25) (layer F.Cu) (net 35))
 (segment (start 144.998998 86.141) (end 145.434 86.141) (width 0.25) (layer F.Cu) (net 38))
 (segment (start 143.898998 85.041) (end 144.998998 86.141) (width 0.25) (layer F.Cu) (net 38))
 (segment (start 142.934 85.041) (end 143.898998 85.041) (width 0.25) (layer F.Cu) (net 38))
 (segment (start 146.824 86.741) (end 146.224 86.141) (width 0.25) (layer F.Cu) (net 38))
 (segment (start 146.224 86.141) (end 145.434 86.141) (width 0.25) (layer F.Cu) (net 38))
 (segment (start 148.336 86.741) (end 146.824 86.741) (width 0.25) (layer F.Cu) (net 38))
 (segment (start 141.98 98.584) (end 142.1195 98.7235) (width 0.25) (layer F.Cu) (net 38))
 (segment (start 140.0055 98.584) (end 141.98 98.584) (width 0.25) (layer F.Cu) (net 38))
 (via (at 145.452 97.9805) (size 0.8) (drill 0.4) (layers F.Cu B.Cu) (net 38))
 (segment (start 145.452001 97.9805) (end 145.452 97.9805) (width 0.25) (layer F.Cu) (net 38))
 (segment (start 149.848 86.741) (end 149.923001 86.816001) (width 0.25) (layer F.Cu) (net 38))
 (segment (start 149.923001 86.816001) (end 149.923001 91.827001) (width 0.25) (layer F.Cu) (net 38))
 (segment (start 149.923001 91.827001) (end 147.718878 94.031124) (width 0.25) (layer F.Cu) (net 38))
 (segment (start 147.718878 95.713623) (end 145.452001 97.9805) (width 0.25) (layer F.Cu) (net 38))
 (segment (start 148.336 86.741) (end 149.848 86.741) (width 0.25) (layer F.Cu) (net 38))
 (segment (start 147.718878 94.031124) (end 147.718878 95.713623) (width 0.25) (layer F.Cu) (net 38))
 (via (at 141.4145 97.7265) (size 0.8) (drill 0.4) (layers F.Cu B.Cu) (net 38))
 (segment (start 145.452 97.9805) (end 141.6685 97.9805) (width 0.25) (layer B.Cu) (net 38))
 (segment (start 141.6685 97.9805) (end 141.4145 97.7265) (width 0.25) (layer B.Cu) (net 38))
 (segment (start 141.4145 98.0185) (end 142.1195 98.7235) (width 0.25) (layer F.Cu) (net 38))
 (segment (start 141.4145 97.7265) (end 141.4145 98.0185) (width 0.25) (layer F.Cu) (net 38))
 (segment (start 133.184 93.964) (end 133.223 94.003) (width 0.25) (layer F.Cu) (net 9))
 (segment (start 133.184 92.041) (end 133.184 93.964) (width 0.25) (layer F.Cu) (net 9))
 (segment (start 133.86801 94.629778) (end 133.86801 97.48251) (width 0.25) (layer F.Cu) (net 9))
 (segment (start 133.27799 94.35299) (end 133.591222 94.35299) (width 0.25) (layer F.Cu) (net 9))
 (segment (start 133.86801 97.48251) (end 134.3025 97.917) (width 0.25) (layer F.Cu) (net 9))
 (segment (start 133.223 94.298) (end 133.27799 94.35299) (width 0.25) (layer F.Cu) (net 9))
 (segment (start 133.591222 94.35299) (end 133.86801 94.629778) (width 0.25) (layer F.Cu) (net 9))
 (segment (start 133.223 94.003) (end 133.223 94.298) (width 0.25) (layer F.Cu) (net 9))
 (segment (start 147.963 84.709) (end 148.463 84.709) (width 0.25) (layer F.Cu) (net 49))
 (segment (start 147.836 84.709) (end 148.336 84.709) (width 0.25) (layer F.Cu) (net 49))
 (segment (start 145.968 82.841) (end 147.836 84.709) (width 0.25) (layer F.Cu) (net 49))
 (segment (start 145.434 82.841) (end 145.968 82.841) (width 0.25) (layer F.Cu) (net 49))
 (segment (start 140.554 94.038) (end 140.739 93.853) (width 0.25) (layer F.Cu) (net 6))
 (segment (start 139.384 94.038) (end 140.554 94.038) (width 0.25) (layer F.Cu) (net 6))
 (segment (start 137.799 93.853) (end 137.984 94.038) (width 0.25) (layer F.Cu) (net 8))
 (segment (start 136.629 93.853) (end 137.799 93.853) (width 0.25) (layer F.Cu) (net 8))
 (segment (start 137.926 94.996) (end 137.984 94.938) (width 0.25) (layer F.Cu) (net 4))
 (segment (start 136.629 94.996) (end 137.926 94.996) (width 0.25) (layer F.Cu) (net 4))
 (segment (start 135.384 93.578) (end 135.659 93.853) (width 0.25) (layer F.Cu) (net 7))
 (segment (start 135.384 92.041) (end 135.384 93.578) (width 0.25) (layer F.Cu) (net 7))
 (segment (start 141.709 92.316) (end 141.984 92.041) (width 0.25) (layer F.Cu) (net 5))
 (segment (start 141.709 93.853) (end 141.709 92.316) (width 0.25) (layer F.Cu) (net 5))
 (segment (start 135.364 94.996) (end 135.659 94.996) (width 0.25) (layer F.Cu) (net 3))
 (segment (start 134.284 93.916) (end 135.364 94.996) (width 0.25) (layer F.Cu) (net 3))
 (segment (start 134.284 92.041) (end 134.284 93.916) (width 0.25) (layer F.Cu) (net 3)))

